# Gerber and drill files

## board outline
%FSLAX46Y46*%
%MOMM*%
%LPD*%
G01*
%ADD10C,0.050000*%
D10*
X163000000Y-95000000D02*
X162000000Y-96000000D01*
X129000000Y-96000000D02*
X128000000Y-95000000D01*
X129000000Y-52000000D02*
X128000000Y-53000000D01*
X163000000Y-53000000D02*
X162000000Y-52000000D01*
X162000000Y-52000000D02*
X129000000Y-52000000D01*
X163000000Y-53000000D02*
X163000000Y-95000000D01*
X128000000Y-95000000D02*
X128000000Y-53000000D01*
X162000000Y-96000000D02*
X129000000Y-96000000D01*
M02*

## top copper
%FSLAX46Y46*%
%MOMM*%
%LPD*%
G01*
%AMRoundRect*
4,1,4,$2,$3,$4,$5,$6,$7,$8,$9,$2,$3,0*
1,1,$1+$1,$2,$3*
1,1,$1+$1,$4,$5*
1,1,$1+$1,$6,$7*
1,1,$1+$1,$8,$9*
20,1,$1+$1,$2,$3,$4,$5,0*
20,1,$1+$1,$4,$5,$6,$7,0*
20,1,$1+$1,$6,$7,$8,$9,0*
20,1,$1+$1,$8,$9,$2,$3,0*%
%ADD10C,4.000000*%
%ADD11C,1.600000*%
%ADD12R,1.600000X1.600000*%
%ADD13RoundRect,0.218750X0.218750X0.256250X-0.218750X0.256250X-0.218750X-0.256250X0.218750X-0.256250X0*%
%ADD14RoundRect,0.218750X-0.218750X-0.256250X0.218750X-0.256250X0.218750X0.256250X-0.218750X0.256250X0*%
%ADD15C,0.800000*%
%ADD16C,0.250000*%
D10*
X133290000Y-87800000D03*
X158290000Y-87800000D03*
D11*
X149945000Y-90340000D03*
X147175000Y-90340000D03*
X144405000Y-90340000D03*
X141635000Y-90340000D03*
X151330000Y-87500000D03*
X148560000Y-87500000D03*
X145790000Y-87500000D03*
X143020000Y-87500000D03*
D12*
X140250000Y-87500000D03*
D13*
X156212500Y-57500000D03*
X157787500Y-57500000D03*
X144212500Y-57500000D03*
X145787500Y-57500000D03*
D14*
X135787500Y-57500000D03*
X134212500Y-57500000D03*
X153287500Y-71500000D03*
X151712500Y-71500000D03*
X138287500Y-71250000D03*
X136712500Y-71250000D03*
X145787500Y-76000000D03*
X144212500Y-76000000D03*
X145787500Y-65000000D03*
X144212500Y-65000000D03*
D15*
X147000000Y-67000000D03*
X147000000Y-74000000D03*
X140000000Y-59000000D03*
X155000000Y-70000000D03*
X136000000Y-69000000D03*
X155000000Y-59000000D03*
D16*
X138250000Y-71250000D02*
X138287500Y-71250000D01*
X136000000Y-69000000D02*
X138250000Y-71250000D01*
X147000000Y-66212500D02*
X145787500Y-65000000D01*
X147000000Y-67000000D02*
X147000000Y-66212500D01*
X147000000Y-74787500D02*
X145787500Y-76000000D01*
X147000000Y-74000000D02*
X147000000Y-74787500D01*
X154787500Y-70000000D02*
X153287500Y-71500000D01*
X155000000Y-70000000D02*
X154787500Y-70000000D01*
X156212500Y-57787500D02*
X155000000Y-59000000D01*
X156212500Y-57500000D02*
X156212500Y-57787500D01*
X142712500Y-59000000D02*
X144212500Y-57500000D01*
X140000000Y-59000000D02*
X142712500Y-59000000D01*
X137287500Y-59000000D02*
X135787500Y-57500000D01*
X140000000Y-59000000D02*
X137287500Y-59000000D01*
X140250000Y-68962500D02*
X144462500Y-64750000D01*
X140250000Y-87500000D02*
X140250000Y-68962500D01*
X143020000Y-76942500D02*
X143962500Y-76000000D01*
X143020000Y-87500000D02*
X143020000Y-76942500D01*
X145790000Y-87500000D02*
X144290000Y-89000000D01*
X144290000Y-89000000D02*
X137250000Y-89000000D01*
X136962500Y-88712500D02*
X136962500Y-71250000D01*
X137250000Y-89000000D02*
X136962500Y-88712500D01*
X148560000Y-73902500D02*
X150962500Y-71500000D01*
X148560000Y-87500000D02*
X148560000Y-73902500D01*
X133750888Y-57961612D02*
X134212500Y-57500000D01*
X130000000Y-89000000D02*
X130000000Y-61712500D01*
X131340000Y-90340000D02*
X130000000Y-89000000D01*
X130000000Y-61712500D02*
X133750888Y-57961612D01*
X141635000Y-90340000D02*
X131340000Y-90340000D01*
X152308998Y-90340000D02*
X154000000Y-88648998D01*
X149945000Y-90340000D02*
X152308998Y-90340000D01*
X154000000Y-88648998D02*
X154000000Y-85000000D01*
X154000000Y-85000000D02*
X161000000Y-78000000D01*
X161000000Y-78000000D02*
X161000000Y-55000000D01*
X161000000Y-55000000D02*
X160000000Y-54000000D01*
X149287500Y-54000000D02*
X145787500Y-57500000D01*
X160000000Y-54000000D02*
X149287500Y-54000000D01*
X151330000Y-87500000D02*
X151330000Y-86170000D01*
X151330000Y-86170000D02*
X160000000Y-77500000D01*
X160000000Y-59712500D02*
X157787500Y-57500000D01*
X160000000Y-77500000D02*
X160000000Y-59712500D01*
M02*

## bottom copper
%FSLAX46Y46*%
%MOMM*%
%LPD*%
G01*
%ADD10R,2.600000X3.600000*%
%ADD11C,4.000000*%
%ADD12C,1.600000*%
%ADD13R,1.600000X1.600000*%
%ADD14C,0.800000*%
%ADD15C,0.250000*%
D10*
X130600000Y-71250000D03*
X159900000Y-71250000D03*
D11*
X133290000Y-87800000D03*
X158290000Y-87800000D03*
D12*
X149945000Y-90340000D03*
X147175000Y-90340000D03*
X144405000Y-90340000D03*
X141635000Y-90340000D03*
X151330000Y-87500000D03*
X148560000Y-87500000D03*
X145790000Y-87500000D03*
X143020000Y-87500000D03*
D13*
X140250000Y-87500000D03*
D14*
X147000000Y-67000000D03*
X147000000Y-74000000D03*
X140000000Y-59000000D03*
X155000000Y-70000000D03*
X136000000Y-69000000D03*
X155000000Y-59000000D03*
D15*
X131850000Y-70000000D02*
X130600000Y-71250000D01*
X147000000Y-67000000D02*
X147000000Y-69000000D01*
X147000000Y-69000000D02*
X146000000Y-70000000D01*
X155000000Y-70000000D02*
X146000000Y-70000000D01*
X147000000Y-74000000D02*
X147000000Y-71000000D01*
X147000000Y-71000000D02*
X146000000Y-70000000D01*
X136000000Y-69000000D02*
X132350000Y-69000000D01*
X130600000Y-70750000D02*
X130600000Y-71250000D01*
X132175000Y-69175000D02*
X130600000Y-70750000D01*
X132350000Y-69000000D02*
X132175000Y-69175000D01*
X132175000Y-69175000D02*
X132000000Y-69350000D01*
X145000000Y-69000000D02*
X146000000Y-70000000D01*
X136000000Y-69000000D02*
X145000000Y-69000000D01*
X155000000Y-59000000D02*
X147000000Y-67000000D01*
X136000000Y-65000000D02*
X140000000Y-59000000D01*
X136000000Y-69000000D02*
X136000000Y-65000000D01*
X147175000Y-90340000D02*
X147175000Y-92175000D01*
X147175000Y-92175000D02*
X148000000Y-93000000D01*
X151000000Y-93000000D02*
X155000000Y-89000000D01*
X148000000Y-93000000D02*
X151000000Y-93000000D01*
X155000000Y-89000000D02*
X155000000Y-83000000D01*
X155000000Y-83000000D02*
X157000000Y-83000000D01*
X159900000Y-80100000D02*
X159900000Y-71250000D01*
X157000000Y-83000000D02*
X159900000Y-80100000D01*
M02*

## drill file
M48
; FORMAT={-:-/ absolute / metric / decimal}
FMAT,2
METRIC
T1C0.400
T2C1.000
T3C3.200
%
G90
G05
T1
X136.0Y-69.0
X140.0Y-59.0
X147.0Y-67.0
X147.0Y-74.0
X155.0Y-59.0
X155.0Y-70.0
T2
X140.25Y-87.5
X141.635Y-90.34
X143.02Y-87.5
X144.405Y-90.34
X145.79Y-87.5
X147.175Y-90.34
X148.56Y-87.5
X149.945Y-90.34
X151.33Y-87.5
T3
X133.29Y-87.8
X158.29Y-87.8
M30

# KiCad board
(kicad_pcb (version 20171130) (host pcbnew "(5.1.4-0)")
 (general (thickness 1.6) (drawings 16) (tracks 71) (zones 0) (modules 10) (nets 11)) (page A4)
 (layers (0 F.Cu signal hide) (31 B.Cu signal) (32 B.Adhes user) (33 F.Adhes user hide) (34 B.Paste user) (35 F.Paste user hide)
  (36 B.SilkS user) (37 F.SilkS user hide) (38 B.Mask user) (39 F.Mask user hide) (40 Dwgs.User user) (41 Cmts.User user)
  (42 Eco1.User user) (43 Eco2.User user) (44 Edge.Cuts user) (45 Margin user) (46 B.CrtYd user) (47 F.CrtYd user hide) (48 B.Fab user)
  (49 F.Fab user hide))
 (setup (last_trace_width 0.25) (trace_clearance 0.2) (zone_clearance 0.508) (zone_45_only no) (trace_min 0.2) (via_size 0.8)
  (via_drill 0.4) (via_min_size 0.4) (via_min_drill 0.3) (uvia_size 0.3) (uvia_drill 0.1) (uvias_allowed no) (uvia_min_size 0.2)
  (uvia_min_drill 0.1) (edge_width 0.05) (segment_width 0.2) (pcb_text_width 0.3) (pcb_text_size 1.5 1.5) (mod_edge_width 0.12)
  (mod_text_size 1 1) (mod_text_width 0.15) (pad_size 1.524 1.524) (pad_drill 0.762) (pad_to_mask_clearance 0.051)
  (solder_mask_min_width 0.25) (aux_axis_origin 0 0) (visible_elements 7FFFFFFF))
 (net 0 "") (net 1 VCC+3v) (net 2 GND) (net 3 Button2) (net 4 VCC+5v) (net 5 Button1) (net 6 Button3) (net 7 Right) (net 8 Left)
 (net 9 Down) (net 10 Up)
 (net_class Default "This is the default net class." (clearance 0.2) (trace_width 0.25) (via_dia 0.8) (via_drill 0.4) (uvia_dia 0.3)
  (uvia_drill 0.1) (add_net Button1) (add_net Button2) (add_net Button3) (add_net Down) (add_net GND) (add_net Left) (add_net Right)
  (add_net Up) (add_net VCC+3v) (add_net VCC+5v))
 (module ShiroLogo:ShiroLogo (layer B.Cu) (at 155 57.5 270)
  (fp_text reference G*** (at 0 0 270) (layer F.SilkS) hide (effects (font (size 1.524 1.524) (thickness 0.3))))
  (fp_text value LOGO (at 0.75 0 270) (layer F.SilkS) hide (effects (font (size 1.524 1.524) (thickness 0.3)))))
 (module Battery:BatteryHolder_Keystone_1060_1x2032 (layer B.Cu) (at 145.25 71.25)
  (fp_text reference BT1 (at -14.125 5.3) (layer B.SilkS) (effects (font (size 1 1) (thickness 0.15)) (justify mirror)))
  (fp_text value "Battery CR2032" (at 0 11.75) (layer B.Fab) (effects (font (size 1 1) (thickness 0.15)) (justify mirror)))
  (pad 1 smd rect (at -14.65 0 180) (size 2.6 3.6) (layers B.Cu B.Paste B.Mask) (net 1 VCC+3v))
  (pad 2 smd rect (at 14.65 0 180) (size 2.6 3.6) (layers B.Cu B.Paste B.Mask) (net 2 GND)))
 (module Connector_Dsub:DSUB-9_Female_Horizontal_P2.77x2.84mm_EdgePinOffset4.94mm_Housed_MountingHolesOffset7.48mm (layer B.Cu)
  (at 140.25 87.5 180)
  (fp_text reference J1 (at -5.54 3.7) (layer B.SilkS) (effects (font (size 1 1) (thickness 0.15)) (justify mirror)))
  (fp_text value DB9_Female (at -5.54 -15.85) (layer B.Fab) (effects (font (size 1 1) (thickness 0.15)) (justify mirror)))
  (pad 0 thru_hole circle (at 6.96 -0.3 180) (size 4 4) (drill 3.2) (layers *.Cu *.Mask))
  (pad 0 thru_hole circle (at -18.04 -0.3 180) (size 4 4) (drill 3.2) (layers *.Cu *.Mask))
  (pad 9 thru_hole circle (at -9.695 -2.84 180) (size 1.6 1.6) (drill 1) (layers *.Cu *.Mask) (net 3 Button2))
  (pad 8 thru_hole circle (at -6.925 -2.84 180) (size 1.6 1.6) (drill 1) (layers *.Cu *.Mask) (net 2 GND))
  (pad 7 thru_hole circle (at -4.155 -2.84 180) (size 1.6 1.6) (drill 1) (layers *.Cu *.Mask) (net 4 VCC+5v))
  (pad 6 thru_hole circle (at -1.385 -2.84 180) (size 1.6 1.6) (drill 1) (layers *.Cu *.Mask) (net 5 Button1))
  (pad 5 thru_hole circle (at -11.08 0 180) (size 1.6 1.6) (drill 1) (layers *.Cu *.Mask) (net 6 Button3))
  (pad 4 thru_hole circle (at -8.31 0 180) (size 1.6 1.6) (drill 1) (layers *.Cu *.Mask) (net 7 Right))
  (pad 3 thru_hole circle (at -5.54 0 180) (size 1.6 1.6) (drill 1) (layers *.Cu *.Mask) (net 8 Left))
  (pad 2 thru_hole circle (at -2.77 0 180) (size 1.6 1.6) (drill 1) (layers *.Cu *.Mask) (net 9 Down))
  (pad 1 thru_hole rect (at 0 0 180) (size 1.6 1.6) (drill 1) (layers *.Cu *.Mask) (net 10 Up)))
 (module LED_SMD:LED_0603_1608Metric (layer F.Cu) (at 157 57.5 180)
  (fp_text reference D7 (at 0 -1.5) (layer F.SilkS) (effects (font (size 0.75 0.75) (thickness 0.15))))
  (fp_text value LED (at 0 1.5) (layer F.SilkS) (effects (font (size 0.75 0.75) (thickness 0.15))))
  (pad 2 smd roundrect (at 0.7875 0 180) (size 0.875 0.95) (layers F.Cu F.Paste F.Mask) (roundrect_rratio 0.25) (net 1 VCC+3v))
  (pad 1 smd roundrect (at -0.7875 0 180) (size 0.875 0.95) (layers F.Cu F.Paste F.Mask) (roundrect_rratio 0.25) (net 6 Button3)))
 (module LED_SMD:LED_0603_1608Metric (layer F.Cu) (at 145 57.5 180)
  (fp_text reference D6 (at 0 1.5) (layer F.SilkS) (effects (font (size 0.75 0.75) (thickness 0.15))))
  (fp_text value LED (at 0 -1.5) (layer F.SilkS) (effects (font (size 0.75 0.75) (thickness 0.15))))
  (pad 2 smd roundrect (at 0.7875 0 180) (size 0.875 0.95) (layers F.Cu F.Paste F.Mask) (roundrect_rratio 0.25) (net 1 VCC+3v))
  (pad 1 smd roundrect (at -0.7875 0 180) (size 0.875 0.95) (layers F.Cu F.Paste F.Mask) (roundrect_rratio 0.25) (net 3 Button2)))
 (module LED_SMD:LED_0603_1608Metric (layer F.Cu) (at 135 57.5)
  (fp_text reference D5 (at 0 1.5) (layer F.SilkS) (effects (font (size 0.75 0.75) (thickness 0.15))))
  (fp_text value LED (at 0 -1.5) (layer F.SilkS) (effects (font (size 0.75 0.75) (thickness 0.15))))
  (pad 2 smd roundrect (at 0.7875 0) (size 0.875 0.95) (layers F.Cu F.Paste F.Mask) (roundrect_rratio 0.25) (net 1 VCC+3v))
  (pad 1 smd roundrect (at -0.7875 0) (size 0.875 0.95) (layers F.Cu F.Paste F.Mask) (roundrect_rratio 0.25) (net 5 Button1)))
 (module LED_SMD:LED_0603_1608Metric (layer F.Cu) (at 152.5 71.5)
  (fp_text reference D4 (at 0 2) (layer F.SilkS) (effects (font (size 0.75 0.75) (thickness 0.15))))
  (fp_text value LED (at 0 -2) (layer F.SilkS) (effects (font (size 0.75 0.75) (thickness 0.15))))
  (pad 2 smd roundrect (at 0.7875 0) (size 0.875 0.95) (layers F.Cu F.Paste F.Mask) (roundrect_rratio 0.25) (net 1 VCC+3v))
  (pad 1 smd roundrect (at -0.7875 0) (size 0.875 0.95) (layers F.Cu F.Paste F.Mask) (roundrect_rratio 0.25) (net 7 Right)))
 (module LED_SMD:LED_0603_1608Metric (layer F.Cu) (at 137.5 71.25)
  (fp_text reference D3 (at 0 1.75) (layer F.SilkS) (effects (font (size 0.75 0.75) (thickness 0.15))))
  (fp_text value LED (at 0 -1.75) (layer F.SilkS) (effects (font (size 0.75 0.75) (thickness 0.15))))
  (pad 2 smd roundrect (at 0.7875 0) (size 0.875 0.95) (layers F.Cu F.Paste F.Mask) (roundrect_rratio 0.25) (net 1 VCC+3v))
  (pad 1 smd roundrect (at -0.7875 0) (size 0.875 0.95) (layers F.Cu F.Paste F.Mask) (roundrect_rratio 0.25) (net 8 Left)))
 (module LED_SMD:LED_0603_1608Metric (layer F.Cu) (at 145 76)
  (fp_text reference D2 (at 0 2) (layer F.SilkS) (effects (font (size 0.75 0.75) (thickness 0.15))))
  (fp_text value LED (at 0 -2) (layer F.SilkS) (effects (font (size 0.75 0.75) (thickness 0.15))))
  (pad 2 smd roundrect (at 0.7875 0) (size 0.875 0.95) (layers F.Cu F.Paste F.Mask) (roundrect_rratio 0.25) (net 1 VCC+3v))
  (pad 1 smd roundrect (at -0.7875 0) (size 0.875 0.95) (layers F.Cu F.Paste F.Mask) (roundrect_rratio 0.25) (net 9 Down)))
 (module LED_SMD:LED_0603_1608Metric (layer F.Cu) (at 145 65)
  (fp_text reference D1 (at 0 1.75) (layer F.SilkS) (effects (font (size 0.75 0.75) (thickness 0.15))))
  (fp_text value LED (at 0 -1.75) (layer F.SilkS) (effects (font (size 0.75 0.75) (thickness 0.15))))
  (pad 2 smd roundrect (at 0.7875 0) (size 0.875 0.95) (layers F.Cu F.Paste F.Mask) (roundrect_rratio 0.25) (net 1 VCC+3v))
  (pad 1 smd roundrect (at -0.7875 0) (size 0.875 0.95) (layers F.Cu F.Paste F.Mask) (roundrect_rratio 0.25) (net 10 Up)))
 (gr_line (start 163 95) (end 162 96) (layer Edge.Cuts) (width 0.05))
 (gr_line (start 129 96) (end 128 95) (layer Edge.Cuts) (width 0.05))
 (gr_line (start 129 52) (end 128 53) (layer Edge.Cuts) (width 0.05))
 (gr_line (start 163 53) (end 162 52) (layer Edge.Cuts) (width 0.05))
 (gr_line (start 162 52) (end 129 52) (layer Edge.Cuts) (width 0.05))
 (gr_line (start 163 53) (end 163 95) (layer Edge.Cuts) (width 0.05))
 (gr_line (start 128 95) (end 128 53) (layer Edge.Cuts) (width 0.05))
 (gr_line (start 162 96) (end 129 96) (layer Edge.Cuts) (width 0.05))
 (via (at 147 67) (size 0.8) (drill 0.4) (layers F.Cu B.Cu) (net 1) (status 1000000))
 (via (at 147 74) (size 0.8) (drill 0.4) (layers F.Cu B.Cu) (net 1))
 (via (at 140 59) (size 0.8) (drill 0.4) (layers F.Cu B.Cu) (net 1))
 (via (at 155 70) (size 0.8) (drill 0.4) (layers F.Cu B.Cu) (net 1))
 (segment (start 131.85 70) (end 130.6 71.25) (width 0.25) (layer B.Cu) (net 1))
 (via (at 136 69) (size 0.8) (drill 0.4) (layers F.Cu B.Cu) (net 1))
 (segment (start 147 67) (end 147 69) (width 0.25) (layer B.Cu) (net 1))
 (segment (start 147 69) (end 146 70) (width 0.25) (layer B.Cu) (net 1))
 (segment (start 155 70) (end 146 70) (width 0.25) (layer B.Cu) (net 1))
 (segment (start 147 74) (end 147 71) (width 0.25) (layer B.Cu) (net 1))
 (segment (start 147 71) (end 146 70) (width 0.25) (layer B.Cu) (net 1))
 (segment (start 136 69) (end 132.35 69) (width 0.25) (layer B.Cu) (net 1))
 (segment (start 130.6 70.75) (end 130.6 71.25) (width 0.25) (layer B.Cu) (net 1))
 (segment (start 132.175 69.175) (end 130.6 70.75) (width 0.25) (layer B.Cu) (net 1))
 (segment (start 132.35 69) (end 132.175 69.175) (width 0.25) (layer B.Cu) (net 1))
 (segment (start 132.175 69.175) (end 132 69.35) (width 0.25) (layer B.Cu) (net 1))
 (segment (start 145 69) (end 146 70) (width 0.25) (layer B.Cu) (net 1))
 (segment (start 136 69) (end 145 69) (width 0.25) (layer B.Cu) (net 1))
 (segment (start 138.25 71.25) (end 138.2875 71.25) (width 0.25) (layer F.Cu) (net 1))
 (segment (start 136 69) (end 138.25 71.25) (width 0.25) (layer F.Cu) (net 1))
 (segment (start 147 66.2125) (end 145.7875 65) (width 0.25) (layer F.Cu) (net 1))
 (segment (start 147 67) (end 147 66.2125) (width 0.25) (layer F.Cu) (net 1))
 (segment (start 147 74.7875) (end 145.7875 76) (width 0.25) (layer F.Cu) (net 1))
 (segment (start 147 74) (end 147 74.7875) (width 0.25) (layer F.Cu) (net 1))
 (segment (start 154.7875 70) (end 153.2875 71.5) (width 0.25) (layer F.Cu) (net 1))
 (segment (start 155 70) (end 154.7875 70) (width 0.25) (layer F.Cu) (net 1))
 (via (at 155 59) (size 0.8) (drill 0.4) (layers F.Cu B.Cu) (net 1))
 (segment (start 155 59) (end 147 67) (width 0.25) (layer B.Cu) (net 1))
 (segment (start 156.2125 57.7875) (end 155 59) (width 0.25) (layer F.Cu) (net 1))
 (segment (start 156.2125 57.5) (end 156.2125 57.7875) (width 0.25) (layer F.Cu) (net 1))
 (segment (start 136 65) (end 140 59) (width 0.25) (layer B.Cu) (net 1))
 (segment (start 136 69) (end 136 65) (width 0.25) (layer B.Cu) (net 1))
 (segment (start 142.7125 59) (end 144.2125 57.5) (width 0.25) (layer F.Cu) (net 1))
 (segment (start 140 59) (end 142.7125 59) (width 0.25) (layer F.Cu) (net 1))
 (segment (start 137.2875 59) (end 135.7875 57.5) (width 0.25) (layer F.Cu) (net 1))
 (segment (start 140 59) (end 137.2875 59) (width 0.25) (layer F.Cu) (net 1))
 (segment (start 147.175 90.34) (end 147.175 92.175) (width 0.25) (layer B.Cu) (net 2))
 (segment (start 147.175 92.175) (end 148 93) (width 0.25) (layer B.Cu) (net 2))
 (segment (start 151 93) (end 155 89) (width 0.25) (layer B.Cu) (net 2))
 (segment (start 148 93) (end 151 93) (width 0.25) (layer B.Cu) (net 2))
 (segment (start 155 89) (end 155 83) (width 0.25) (layer B.Cu) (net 2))
 (segment (start 155 83) (end 157 83) (width 0.25) (layer B.Cu) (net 2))
 (segment (start 159.9 80.1) (end 159.9 71.25) (width 0.25) (layer B.Cu) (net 2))
 (segment (start 157 83) (end 159.9 80.1) (width 0.25) (layer B.Cu) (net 2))
 (segment (start 140.25 68.9625) (end 144.4625 64.75) (width 0.25) (layer F.Cu) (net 10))
 (segment (start 140.25 87.5) (end 140.25 68.9625) (width 0.25) (layer F.Cu) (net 10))
 (segment (start 143.02 76.9425) (end 143.9625 76) (width 0.25) (layer F.Cu) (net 9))
 (segment (start 143.02 87.5) (end 143.02 76.9425) (width 0.25) (layer F.Cu) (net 9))
 (segment (start 145.79 87.5) (end 144.29 89) (width 0.25) (layer F.Cu) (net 8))
 (segment (start 144.29 89) (end 137.25 89) (width 0.25) (layer F.Cu) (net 8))
 (segment (start 136.9625 88.7125) (end 136.9625 71.25) (width 0.25) (layer F.Cu) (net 8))
 (segment (start 137.25 89) (end 136.9625 88.7125) (width 0.25) (layer F.Cu) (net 8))
 (segment (start 148.56 73.9025) (end 150.9625 71.5) (width 0.25) (layer F.Cu) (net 7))
 (segment (start 148.56 87.5) (end 148.56 73.9025) (width 0.25) (layer F.Cu) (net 7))
 (segment (start 133.750888 57.961612) (end 134.2125 57.5) (width 0.25) (layer F.Cu) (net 5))
 (segment (start 130 89) (end 130 61.7125) (width 0.25) (layer F.Cu) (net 5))
 (segment (start 131.34 90.34) (end 130 89) (width 0.25) (layer F.Cu) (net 5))
 (segment (start 130 61.7125) (end 133.750888 57.961612) (width 0.25) (layer F.Cu) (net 5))
 (segment (start 141.635 90.34) (end 131.34 90.34) (width 0.25) (layer F.Cu) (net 5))
 (segment (start 152.308998 90.34) (end 154 88.648998) (width 0.25) (layer F.Cu) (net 3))
 (segment (start 149.945 90.34) (end 152.308998 90.34) (width 0.25) (layer F.Cu) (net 3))
 (segment (start 154 88.648998) (end 154 85) (width 0.25) (layer F.Cu) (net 3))
 (segment (start 154 85) (end 161 78) (width 0.25) (layer F.Cu) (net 3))
 (segment (start 161 78) (end 161 55) (width 0.25) (layer F.Cu) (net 3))
 (segment (start 161 55) (end 160 54) (width 0.25) (layer F.Cu) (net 3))
 (segment (start 149.2875 54) (end 145.7875 57.5) (width 0.25) (layer F.Cu) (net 3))
 (segment (start 160 54) (end 149.2875 54) (width 0.25) (layer F.Cu) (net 3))
 (segment (start 151.33 87.5) (end 151.33 86.17) (width 0.25) (layer F.Cu) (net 6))
 (segment (start 151.33 86.17) (end 160 77.5) (width 0.25) (layer F.Cu) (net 6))
 (segment (start 160 59.7125) (end 157.7875 57.5) (width 0.25) (layer F.Cu) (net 6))
 (segment (start 160 77.5) (end 160 59.7125) (width 0.25) (layer F.Cu) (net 6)))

